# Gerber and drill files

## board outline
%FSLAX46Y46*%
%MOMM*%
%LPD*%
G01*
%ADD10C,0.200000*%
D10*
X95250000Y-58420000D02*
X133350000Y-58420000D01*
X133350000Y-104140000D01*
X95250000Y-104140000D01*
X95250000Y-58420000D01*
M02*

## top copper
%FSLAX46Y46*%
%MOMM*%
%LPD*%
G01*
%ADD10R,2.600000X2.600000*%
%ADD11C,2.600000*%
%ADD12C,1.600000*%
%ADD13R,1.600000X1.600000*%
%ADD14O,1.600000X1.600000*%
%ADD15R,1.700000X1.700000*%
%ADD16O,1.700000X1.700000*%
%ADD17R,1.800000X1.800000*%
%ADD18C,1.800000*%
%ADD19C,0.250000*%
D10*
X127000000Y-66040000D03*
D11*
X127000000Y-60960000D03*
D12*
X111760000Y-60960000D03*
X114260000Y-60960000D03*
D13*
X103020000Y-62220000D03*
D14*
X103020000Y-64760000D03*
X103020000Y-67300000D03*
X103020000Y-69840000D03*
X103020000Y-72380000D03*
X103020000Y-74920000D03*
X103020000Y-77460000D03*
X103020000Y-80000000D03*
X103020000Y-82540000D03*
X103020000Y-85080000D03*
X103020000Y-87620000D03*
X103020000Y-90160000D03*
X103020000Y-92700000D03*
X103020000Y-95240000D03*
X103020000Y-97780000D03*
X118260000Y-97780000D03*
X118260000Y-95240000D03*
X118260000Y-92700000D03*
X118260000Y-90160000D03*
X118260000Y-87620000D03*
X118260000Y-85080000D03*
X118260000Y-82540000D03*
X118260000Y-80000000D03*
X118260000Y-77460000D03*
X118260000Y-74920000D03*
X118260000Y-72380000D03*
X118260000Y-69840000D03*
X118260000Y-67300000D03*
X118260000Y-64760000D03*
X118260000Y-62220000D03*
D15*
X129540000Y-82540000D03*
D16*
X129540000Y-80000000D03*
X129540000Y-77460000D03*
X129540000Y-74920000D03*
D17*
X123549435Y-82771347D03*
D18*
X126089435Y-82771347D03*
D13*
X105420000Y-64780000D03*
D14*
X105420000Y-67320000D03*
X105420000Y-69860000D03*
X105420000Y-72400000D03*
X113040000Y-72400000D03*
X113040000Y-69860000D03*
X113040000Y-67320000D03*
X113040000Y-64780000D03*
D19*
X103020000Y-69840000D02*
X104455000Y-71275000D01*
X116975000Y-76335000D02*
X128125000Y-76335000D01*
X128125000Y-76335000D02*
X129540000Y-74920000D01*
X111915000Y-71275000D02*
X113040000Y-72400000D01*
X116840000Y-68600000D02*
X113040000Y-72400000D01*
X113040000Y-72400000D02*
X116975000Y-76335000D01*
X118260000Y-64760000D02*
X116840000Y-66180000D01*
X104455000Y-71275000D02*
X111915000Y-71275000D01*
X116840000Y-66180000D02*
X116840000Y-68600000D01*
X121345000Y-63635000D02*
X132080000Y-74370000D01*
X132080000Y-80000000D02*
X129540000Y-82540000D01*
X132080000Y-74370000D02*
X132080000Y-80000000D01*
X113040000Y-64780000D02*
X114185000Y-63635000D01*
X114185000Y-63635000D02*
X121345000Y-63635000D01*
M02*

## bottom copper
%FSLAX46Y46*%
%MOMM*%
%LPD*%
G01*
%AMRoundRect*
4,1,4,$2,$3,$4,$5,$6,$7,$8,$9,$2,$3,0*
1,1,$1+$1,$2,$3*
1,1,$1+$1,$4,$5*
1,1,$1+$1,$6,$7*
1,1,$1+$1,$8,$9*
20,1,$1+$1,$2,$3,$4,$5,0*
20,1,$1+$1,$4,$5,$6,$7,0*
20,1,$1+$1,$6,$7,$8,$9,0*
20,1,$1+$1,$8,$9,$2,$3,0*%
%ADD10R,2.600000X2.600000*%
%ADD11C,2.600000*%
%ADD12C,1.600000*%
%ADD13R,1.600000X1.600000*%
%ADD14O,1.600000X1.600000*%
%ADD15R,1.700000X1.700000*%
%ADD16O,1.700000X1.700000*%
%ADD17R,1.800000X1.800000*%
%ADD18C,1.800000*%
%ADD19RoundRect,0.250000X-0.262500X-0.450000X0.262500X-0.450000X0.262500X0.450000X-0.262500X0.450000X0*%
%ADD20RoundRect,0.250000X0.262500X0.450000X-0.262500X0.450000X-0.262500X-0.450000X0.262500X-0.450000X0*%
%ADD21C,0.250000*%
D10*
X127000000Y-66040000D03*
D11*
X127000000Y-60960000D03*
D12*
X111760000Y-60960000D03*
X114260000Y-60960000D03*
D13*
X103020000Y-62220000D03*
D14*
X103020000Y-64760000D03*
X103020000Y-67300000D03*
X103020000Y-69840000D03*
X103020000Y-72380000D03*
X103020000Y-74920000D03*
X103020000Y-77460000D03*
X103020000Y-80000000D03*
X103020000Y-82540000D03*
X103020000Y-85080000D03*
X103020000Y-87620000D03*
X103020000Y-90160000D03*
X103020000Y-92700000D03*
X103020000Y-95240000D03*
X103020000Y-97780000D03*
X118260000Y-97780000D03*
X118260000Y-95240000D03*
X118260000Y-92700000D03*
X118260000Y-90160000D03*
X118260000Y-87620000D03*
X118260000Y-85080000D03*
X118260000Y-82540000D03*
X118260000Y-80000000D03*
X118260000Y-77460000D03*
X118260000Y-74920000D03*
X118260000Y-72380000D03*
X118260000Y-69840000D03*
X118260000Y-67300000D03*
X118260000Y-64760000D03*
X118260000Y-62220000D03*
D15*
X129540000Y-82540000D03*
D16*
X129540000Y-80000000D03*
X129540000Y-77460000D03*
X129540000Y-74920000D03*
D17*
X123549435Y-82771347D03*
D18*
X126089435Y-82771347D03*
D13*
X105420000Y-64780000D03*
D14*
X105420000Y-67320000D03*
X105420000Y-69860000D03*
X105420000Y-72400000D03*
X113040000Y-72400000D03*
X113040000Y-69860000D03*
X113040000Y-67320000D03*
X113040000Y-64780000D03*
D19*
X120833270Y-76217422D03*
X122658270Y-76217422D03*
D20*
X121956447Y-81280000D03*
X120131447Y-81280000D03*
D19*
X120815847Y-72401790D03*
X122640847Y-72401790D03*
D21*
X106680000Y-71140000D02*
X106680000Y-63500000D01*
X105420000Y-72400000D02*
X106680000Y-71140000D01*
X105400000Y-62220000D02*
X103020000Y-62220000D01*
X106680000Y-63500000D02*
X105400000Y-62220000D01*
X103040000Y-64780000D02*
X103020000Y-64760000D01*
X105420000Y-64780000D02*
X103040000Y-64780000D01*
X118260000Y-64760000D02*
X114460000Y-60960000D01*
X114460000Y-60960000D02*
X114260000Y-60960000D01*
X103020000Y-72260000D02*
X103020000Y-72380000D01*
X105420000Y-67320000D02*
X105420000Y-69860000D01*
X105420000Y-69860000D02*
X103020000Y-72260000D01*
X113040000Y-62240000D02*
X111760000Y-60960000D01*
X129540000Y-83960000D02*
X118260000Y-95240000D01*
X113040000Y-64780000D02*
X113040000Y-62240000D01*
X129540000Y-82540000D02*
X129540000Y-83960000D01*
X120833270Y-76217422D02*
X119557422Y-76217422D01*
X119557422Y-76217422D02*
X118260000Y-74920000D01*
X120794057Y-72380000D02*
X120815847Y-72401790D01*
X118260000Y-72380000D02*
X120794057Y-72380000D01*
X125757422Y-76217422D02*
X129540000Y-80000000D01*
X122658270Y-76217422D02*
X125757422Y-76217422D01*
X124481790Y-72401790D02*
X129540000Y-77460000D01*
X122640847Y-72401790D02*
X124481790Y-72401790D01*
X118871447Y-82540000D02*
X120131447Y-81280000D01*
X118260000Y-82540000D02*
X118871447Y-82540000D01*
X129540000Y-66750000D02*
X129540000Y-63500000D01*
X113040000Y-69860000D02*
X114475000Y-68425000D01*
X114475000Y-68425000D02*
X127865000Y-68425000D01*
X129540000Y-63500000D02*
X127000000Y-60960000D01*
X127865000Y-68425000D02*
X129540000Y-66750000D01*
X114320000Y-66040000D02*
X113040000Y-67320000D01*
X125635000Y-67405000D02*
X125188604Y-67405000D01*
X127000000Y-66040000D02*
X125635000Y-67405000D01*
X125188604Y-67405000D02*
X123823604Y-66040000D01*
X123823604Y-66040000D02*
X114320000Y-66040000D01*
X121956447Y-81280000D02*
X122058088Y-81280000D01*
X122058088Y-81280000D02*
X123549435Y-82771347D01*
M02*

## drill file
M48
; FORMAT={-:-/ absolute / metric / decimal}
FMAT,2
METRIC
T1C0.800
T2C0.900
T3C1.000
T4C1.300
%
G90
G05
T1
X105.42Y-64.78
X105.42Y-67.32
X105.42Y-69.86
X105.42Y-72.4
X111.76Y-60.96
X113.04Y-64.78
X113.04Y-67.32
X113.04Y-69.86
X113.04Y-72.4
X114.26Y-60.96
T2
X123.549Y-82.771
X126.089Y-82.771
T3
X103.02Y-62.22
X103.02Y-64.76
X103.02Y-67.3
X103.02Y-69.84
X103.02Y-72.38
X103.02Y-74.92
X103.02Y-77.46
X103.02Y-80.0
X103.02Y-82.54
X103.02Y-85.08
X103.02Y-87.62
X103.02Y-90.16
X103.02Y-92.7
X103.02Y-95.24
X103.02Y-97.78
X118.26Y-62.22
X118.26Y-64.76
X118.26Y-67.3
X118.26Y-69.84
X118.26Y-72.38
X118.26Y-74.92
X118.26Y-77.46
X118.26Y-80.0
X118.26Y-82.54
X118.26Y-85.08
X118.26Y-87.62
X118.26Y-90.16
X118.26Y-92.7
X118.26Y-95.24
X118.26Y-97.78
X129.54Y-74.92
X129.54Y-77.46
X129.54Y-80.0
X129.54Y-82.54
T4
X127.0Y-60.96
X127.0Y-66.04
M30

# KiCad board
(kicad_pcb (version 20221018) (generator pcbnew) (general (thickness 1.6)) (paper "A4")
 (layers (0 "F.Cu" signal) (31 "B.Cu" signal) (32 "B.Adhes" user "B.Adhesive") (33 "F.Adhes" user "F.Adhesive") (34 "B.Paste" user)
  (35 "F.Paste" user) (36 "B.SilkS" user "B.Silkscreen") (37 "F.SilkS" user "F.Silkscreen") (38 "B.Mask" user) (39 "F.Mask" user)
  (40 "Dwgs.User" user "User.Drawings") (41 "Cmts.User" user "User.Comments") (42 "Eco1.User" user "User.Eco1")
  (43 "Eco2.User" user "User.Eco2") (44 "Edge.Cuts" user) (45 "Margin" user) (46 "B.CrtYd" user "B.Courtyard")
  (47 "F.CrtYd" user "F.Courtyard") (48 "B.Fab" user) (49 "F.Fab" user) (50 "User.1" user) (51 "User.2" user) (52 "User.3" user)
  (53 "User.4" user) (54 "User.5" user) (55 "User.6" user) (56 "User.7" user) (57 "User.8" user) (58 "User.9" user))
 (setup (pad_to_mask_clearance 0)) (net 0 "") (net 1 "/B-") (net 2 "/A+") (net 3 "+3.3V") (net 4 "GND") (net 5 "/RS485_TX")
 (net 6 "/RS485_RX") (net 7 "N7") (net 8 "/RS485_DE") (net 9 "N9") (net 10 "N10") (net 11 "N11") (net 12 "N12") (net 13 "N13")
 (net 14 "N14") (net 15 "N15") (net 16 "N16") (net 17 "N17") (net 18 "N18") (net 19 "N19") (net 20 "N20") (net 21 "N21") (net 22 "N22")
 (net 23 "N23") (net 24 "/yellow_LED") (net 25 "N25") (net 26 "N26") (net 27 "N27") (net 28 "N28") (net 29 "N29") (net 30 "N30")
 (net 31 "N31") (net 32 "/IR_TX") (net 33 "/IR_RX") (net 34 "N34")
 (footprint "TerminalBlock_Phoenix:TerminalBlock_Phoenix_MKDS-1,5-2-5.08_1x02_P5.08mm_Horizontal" (layer "F.Cu") (at 127 66.04 90)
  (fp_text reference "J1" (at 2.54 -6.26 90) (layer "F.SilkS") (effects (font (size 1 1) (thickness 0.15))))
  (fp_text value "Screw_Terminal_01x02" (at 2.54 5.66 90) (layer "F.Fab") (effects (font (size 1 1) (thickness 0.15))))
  (pad "1" thru_hole rect (at 0 0 90) (size 2.6 2.6) (drill 1.3) (layers "*.Cu" "*.Mask") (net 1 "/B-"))
  (pad "2" thru_hole circle (at 5.08 0 90) (size 2.6 2.6) (drill 1.3) (layers "*.Cu" "*.Mask") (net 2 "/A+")))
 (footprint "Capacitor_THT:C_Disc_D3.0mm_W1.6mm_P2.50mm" (layer "F.Cu") (at 111.76 60.96)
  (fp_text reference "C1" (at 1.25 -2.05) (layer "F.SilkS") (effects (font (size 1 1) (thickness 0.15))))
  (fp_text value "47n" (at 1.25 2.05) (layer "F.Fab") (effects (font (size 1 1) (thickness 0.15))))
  (pad "1" thru_hole circle (at 0 0) (size 1.6 1.6) (drill 0.8) (layers "*.Cu" "*.Mask") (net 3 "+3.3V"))
  (pad "2" thru_hole circle (at 2.5 0) (size 1.6 1.6) (drill 0.8) (layers "*.Cu" "*.Mask") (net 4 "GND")))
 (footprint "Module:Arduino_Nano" (layer "F.Cu") (at 103.02 62.22)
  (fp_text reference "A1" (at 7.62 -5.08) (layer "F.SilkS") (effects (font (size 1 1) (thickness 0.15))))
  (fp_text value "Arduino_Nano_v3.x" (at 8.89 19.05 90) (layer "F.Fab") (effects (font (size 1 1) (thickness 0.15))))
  (pad "1" thru_hole rect (at 0 0) (size 1.6 1.6) (drill 1) (layers "*.Cu" "*.Mask") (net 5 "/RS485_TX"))
  (pad "2" thru_hole oval (at 0 2.54) (size 1.6 1.6) (drill 1) (layers "*.Cu" "*.Mask") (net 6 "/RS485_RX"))
  (pad "3" thru_hole oval (at 0 5.08) (size 1.6 1.6) (drill 1) (layers "*.Cu" "*.Mask") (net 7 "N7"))
  (pad "4" thru_hole oval (at 0 7.62) (size 1.6 1.6) (drill 1) (layers "*.Cu" "*.Mask") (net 4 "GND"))
  (pad "5" thru_hole oval (at 0 10.16) (size 1.6 1.6) (drill 1) (layers "*.Cu" "*.Mask") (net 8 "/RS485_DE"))
  (pad "6" thru_hole oval (at 0 12.7) (size 1.6 1.6) (drill 1) (layers "*.Cu" "*.Mask") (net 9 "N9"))
  (pad "7" thru_hole oval (at 0 15.24) (size 1.6 1.6) (drill 1) (layers "*.Cu" "*.Mask") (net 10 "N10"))
  (pad "8" thru_hole oval (at 0 17.78) (size 1.6 1.6) (drill 1) (layers "*.Cu" "*.Mask") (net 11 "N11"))
  (pad "9" thru_hole oval (at 0 20.32) (size 1.6 1.6) (drill 1) (layers "*.Cu" "*.Mask") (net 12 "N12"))
  (pad "10" thru_hole oval (at 0 22.86) (size 1.6 1.6) (drill 1) (layers "*.Cu" "*.Mask") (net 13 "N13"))
  (pad "11" thru_hole oval (at 0 25.4) (size 1.6 1.6) (drill 1) (layers "*.Cu" "*.Mask") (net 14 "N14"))
  (pad "12" thru_hole oval (at 0 27.94) (size 1.6 1.6) (drill 1) (layers "*.Cu" "*.Mask") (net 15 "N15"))
  (pad "13" thru_hole oval (at 0 30.48) (size 1.6 1.6) (drill 1) (layers "*.Cu" "*.Mask") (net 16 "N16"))
  (pad "14" thru_hole oval (at 0 33.02) (size 1.6 1.6) (drill 1) (layers "*.Cu" "*.Mask") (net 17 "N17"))
  (pad "15" thru_hole oval (at 0 35.56) (size 1.6 1.6) (drill 1) (layers "*.Cu" "*.Mask") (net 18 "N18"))
  (pad "16" thru_hole oval (at 15.24 35.56) (size 1.6 1.6) (drill 1) (layers "*.Cu" "*.Mask") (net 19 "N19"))
  (pad "17" thru_hole oval (at 15.24 33.02) (size 1.6 1.6) (drill 1) (layers "*.Cu" "*.Mask") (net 3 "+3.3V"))
  (pad "18" thru_hole oval (at 15.24 30.48) (size 1.6 1.6) (drill 1) (layers "*.Cu" "*.Mask") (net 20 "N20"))
  (pad "19" thru_hole oval (at 15.24 27.94) (size 1.6 1.6) (drill 1) (layers "*.Cu" "*.Mask") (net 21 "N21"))
  (pad "20" thru_hole oval (at 15.24 25.4) (size 1.6 1.6) (drill 1) (layers "*.Cu" "*.Mask") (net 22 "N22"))
  (pad "21" thru_hole oval (at 15.24 22.86) (size 1.6 1.6) (drill 1) (layers "*.Cu" "*.Mask") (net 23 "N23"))
  (pad "22" thru_hole oval (at 15.24 20.32) (size 1.6 1.6) (drill 1) (layers "*.Cu" "*.Mask") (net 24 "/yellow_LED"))
  (pad "23" thru_hole oval (at 15.24 17.78) (size 1.6 1.6) (drill 1) (layers "*.Cu" "*.Mask") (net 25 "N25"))
  (pad "24" thru_hole oval (at 15.24 15.24) (size 1.6 1.6) (drill 1) (layers "*.Cu" "*.Mask") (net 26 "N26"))
  (pad "25" thru_hole oval (at 15.24 12.7) (size 1.6 1.6) (drill 1) (layers "*.Cu" "*.Mask") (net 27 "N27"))
  (pad "26" thru_hole oval (at 15.24 10.16) (size 1.6 1.6) (drill 1) (layers "*.Cu" "*.Mask") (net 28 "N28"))
  (pad "27" thru_hole oval (at 15.24 7.62) (size 1.6 1.6) (drill 1) (layers "*.Cu" "*.Mask") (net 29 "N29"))
  (pad "28" thru_hole oval (at 15.24 5.08) (size 1.6 1.6) (drill 1) (layers "*.Cu" "*.Mask") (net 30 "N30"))
  (pad "29" thru_hole oval (at 15.24 2.54) (size 1.6 1.6) (drill 1) (layers "*.Cu" "*.Mask") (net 4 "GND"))
  (pad "30" thru_hole oval (at 15.24 0) (size 1.6 1.6) (drill 1) (layers "*.Cu" "*.Mask") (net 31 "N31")))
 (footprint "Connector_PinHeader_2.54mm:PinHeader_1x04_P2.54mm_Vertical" (layer "F.Cu") (at 129.54 82.54 180)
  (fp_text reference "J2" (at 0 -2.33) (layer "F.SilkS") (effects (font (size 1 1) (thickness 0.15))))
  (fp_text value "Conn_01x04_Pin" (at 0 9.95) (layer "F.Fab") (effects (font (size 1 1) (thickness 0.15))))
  (pad "1" thru_hole rect (at 0 0 180) (size 1.7 1.7) (drill 1) (layers "*.Cu" "*.Mask") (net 3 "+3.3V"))
  (pad "2" thru_hole oval (at 0 2.54 180) (size 1.7 1.7) (drill 1) (layers "*.Cu" "*.Mask") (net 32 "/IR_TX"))
  (pad "3" thru_hole oval (at 0 5.08 180) (size 1.7 1.7) (drill 1) (layers "*.Cu" "*.Mask") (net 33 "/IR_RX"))
  (pad "4" thru_hole oval (at 0 7.62 180) (size 1.7 1.7) (drill 1) (layers "*.Cu" "*.Mask") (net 4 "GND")))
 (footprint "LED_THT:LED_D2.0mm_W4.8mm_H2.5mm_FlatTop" (layer "F.Cu") (at 123.549435 82.771347)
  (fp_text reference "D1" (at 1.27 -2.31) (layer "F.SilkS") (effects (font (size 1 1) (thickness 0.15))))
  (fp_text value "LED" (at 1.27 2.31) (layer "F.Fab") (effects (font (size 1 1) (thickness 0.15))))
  (pad "1" thru_hole rect (at 0 0) (size 1.8 1.8) (drill 0.9) (layers "*.Cu" "*.Mask") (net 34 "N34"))
  (pad "2" thru_hole circle (at 2.54 0) (size 1.8 1.8) (drill 0.9) (layers "*.Cu" "*.Mask") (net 3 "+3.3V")))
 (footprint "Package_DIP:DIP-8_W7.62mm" (layer "F.Cu") (at 105.42 64.78)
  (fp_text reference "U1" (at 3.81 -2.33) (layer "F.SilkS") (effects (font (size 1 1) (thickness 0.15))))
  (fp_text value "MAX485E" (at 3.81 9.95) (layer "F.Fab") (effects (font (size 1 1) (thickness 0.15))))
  (pad "1" thru_hole rect (at 0 0) (size 1.6 1.6) (drill 0.8) (layers "*.Cu" "*.Mask") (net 6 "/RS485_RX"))
  (pad "2" thru_hole oval (at 0 2.54) (size 1.6 1.6) (drill 0.8) (layers "*.Cu" "*.Mask") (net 8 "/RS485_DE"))
  (pad "3" thru_hole oval (at 0 5.08) (size 1.6 1.6) (drill 0.8) (layers "*.Cu" "*.Mask") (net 8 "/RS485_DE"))
  (pad "4" thru_hole oval (at 0 7.62) (size 1.6 1.6) (drill 0.8) (layers "*.Cu" "*.Mask") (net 5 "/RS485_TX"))
  (pad "5" thru_hole oval (at 7.62 7.62) (size 1.6 1.6) (drill 0.8) (layers "*.Cu" "*.Mask") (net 4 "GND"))
  (pad "6" thru_hole oval (at 7.62 5.08) (size 1.6 1.6) (drill 0.8) (layers "*.Cu" "*.Mask") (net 2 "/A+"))
  (pad "7" thru_hole oval (at 7.62 2.54) (size 1.6 1.6) (drill 0.8) (layers "*.Cu" "*.Mask") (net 1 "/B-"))
  (pad "8" thru_hole oval (at 7.62 0) (size 1.6 1.6) (drill 0.8) (layers "*.Cu" "*.Mask") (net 3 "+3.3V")))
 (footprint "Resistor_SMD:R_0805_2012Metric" (layer "B.Cu") (at 121.74577 76.217422)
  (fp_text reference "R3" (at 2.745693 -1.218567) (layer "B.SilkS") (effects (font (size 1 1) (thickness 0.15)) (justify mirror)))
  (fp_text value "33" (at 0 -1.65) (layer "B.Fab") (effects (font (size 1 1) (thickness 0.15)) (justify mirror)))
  (pad "1" smd roundrect (at -0.9125 0) (size 1.025 1.4) (layers "B.Cu" "B.Paste" "B.Mask") (roundrect_rratio 0.243902) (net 27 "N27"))
  (pad "2" smd roundrect (at 0.9125 0) (size 1.025 1.4) (layers "B.Cu" "B.Paste" "B.Mask") (roundrect_rratio 0.243902) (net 32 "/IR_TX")))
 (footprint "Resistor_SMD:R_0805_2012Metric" (layer "B.Cu") (at 121.043947 81.28 180)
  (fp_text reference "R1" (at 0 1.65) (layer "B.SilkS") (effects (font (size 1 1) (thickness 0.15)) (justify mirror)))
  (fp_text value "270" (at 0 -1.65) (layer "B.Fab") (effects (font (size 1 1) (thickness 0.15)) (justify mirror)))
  (pad "1" smd roundrect (at -0.9125 0 180) (size 1.025 1.4) (layers "B.Cu" "B.Paste" "B.Mask") (roundrect_rratio 0.243902) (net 34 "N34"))
  (pad "2" smd roundrect (at 0.9125 0 180) (size 1.025 1.4) (layers "B.Cu" "B.Paste" "B.Mask") (roundrect_rratio 0.243902)
   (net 24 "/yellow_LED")))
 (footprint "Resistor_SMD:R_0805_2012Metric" (layer "B.Cu") (at 121.728347 72.40179)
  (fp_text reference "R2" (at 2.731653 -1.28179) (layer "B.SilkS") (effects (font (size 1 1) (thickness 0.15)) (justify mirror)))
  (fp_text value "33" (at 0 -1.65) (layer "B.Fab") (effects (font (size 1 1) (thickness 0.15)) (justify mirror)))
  (pad "1" smd roundrect (at -0.9125 0) (size 1.025 1.4) (layers "B.Cu" "B.Paste" "B.Mask") (roundrect_rratio 0.243902) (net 28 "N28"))
  (pad "2" smd roundrect (at 0.9125 0) (size 1.025 1.4) (layers "B.Cu" "B.Paste" "B.Mask") (roundrect_rratio 0.243902) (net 33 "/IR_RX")))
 (gr_rect (start 95.25 58.42) (end 133.35 104.14) (stroke (width 0.2) (type default)) (fill none) (layer "Edge.Cuts"))
 (segment (start 106.68 71.14) (end 106.68 63.5) (width 0.25) (layer "B.Cu") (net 5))
 (segment (start 105.42 72.4) (end 106.68 71.14) (width 0.25) (layer "B.Cu") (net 5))
 (segment (start 105.4 62.22) (end 103.02 62.22) (width 0.25) (layer "B.Cu") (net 5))
 (segment (start 106.68 63.5) (end 105.4 62.22) (width 0.25) (layer "B.Cu") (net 5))
 (segment (start 103.04 64.78) (end 103.02 64.76) (width 0.25) (layer "B.Cu") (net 6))
 (segment (start 105.42 64.78) (end 103.04 64.78) (width 0.25) (layer "B.Cu") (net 6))
 (segment (start 103.02 69.84) (end 104.455 71.275) (width 0.25) (layer "F.Cu") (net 4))
 (segment (start 116.975 76.335) (end 128.125 76.335) (width 0.25) (layer "F.Cu") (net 4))
 (segment (start 128.125 76.335) (end 129.54 74.92) (width 0.25) (layer "F.Cu") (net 4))
 (segment (start 111.915 71.275) (end 113.04 72.4) (width 0.25) (layer "F.Cu") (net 4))
 (segment (start 116.84 68.6) (end 113.04 72.4) (width 0.25) (layer "F.Cu") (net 4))
 (segment (start 113.04 72.4) (end 116.975 76.335) (width 0.25) (layer "F.Cu") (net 4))
 (segment (start 118.26 64.76) (end 116.84 66.18) (width 0.25) (layer "F.Cu") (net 4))
 (segment (start 104.455 71.275) (end 111.915 71.275) (width 0.25) (layer "F.Cu") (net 4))
 (segment (start 116.84 66.18) (end 116.84 68.6) (width 0.25) (layer "F.Cu") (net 4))
 (segment (start 118.26 64.76) (end 114.46 60.96) (width 0.25) (layer "B.Cu") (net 4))
 (segment (start 114.46 60.96) (end 114.26 60.96) (width 0.25) (layer "B.Cu") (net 4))
 (segment (start 103.02 72.26) (end 103.02 72.38) (width 0.25) (layer "B.Cu") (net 8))
 (segment (start 105.42 67.32) (end 105.42 69.86) (width 0.25) (layer "B.Cu") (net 8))
 (segment (start 105.42 69.86) (end 103.02 72.26) (width 0.25) (layer "B.Cu") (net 8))
 (segment (start 121.345 63.635) (end 132.08 74.37) (width 0.25) (layer "F.Cu") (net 3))
 (segment (start 132.08 80) (end 129.54 82.54) (width 0.25) (layer "F.Cu") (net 3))
 (segment (start 132.08 74.37) (end 132.08 80) (width 0.25) (layer "F.Cu") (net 3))
 (segment (start 113.04 64.78) (end 114.185 63.635) (width 0.25) (layer "F.Cu") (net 3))
 (segment (start 114.185 63.635) (end 121.345 63.635) (width 0.25) (layer "F.Cu") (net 3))
 (segment (start 113.04 62.24) (end 111.76 60.96) (width 0.25) (layer "B.Cu") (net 3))
 (segment (start 129.54 83.96) (end 118.26 95.24) (width 0.25) (layer "B.Cu") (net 3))
 (segment (start 113.04 64.78) (end 113.04 62.24) (width 0.25) (layer "B.Cu") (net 3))
 (segment (start 129.54 82.54) (end 129.54 83.96) (width 0.25) (layer "B.Cu") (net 3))
 (segment (start 120.83327 76.217422) (end 119.557422 76.217422) (width 0.25) (layer "B.Cu") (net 27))
 (segment (start 119.557422 76.217422) (end 118.26 74.92) (width 0.25) (layer "B.Cu") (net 27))
 (segment (start 120.794057 72.38) (end 120.815847 72.40179) (width 0.25) (layer "B.Cu") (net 28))
 (segment (start 118.26 72.38) (end 120.794057 72.38) (width 0.25) (layer "B.Cu") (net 28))
 (segment (start 125.757422 76.217422) (end 129.54 80) (width 0.25) (layer "B.Cu") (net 32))
 (segment (start 122.65827 76.217422) (end 125.757422 76.217422) (width 0.25) (layer "B.Cu") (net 32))
 (segment (start 124.48179 72.40179) (end 129.54 77.46) (width 0.25) (layer "B.Cu") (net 33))
 (segment (start 122.640847 72.40179) (end 124.48179 72.40179) (width 0.25) (layer "B.Cu") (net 33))
 (segment (start 118.871447 82.54) (end 120.131447 81.28) (width 0.25) (layer "B.Cu") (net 24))
 (segment (start 118.26 82.54) (end 118.871447 82.54) (width 0.25) (layer "B.Cu") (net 24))
 (segment (start 129.54 66.75) (end 129.54 63.5) (width 0.25) (layer "B.Cu") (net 2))
 (segment (start 113.04 69.86) (end 114.475 68.425) (width 0.25) (layer "B.Cu") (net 2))
 (segment (start 114.475 68.425) (end 127.865 68.425) (width 0.25) (layer "B.Cu") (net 2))
 (segment (start 129.54 63.5) (end 127 60.96) (width 0.25) (layer "B.Cu") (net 2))
 (segment (start 127.865 68.425) (end 129.54 66.75) (width 0.25) (layer "B.Cu") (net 2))
 (segment (start 114.32 66.04) (end 113.04 67.32) (width 0.25) (layer "B.Cu") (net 1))
 (segment (start 125.635 67.405) (end 125.188604 67.405) (width 0.25) (layer "B.Cu") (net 1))
 (segment (start 127 66.04) (end 125.635 67.405) (width 0.25) (layer "B.Cu") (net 1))
 (segment (start 125.188604 67.405) (end 123.823604 66.04) (width 0.25) (layer "B.Cu") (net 1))
 (segment (start 123.823604 66.04) (end 114.32 66.04) (width 0.25) (layer "B.Cu") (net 1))
 (segment (start 121.956447 81.28) (end 122.058088 81.28) (width 0.25) (layer "B.Cu") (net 34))
 (segment (start 122.058088 81.28) (end 123.549435 82.771347) (width 0.25) (layer "B.Cu") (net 34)))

